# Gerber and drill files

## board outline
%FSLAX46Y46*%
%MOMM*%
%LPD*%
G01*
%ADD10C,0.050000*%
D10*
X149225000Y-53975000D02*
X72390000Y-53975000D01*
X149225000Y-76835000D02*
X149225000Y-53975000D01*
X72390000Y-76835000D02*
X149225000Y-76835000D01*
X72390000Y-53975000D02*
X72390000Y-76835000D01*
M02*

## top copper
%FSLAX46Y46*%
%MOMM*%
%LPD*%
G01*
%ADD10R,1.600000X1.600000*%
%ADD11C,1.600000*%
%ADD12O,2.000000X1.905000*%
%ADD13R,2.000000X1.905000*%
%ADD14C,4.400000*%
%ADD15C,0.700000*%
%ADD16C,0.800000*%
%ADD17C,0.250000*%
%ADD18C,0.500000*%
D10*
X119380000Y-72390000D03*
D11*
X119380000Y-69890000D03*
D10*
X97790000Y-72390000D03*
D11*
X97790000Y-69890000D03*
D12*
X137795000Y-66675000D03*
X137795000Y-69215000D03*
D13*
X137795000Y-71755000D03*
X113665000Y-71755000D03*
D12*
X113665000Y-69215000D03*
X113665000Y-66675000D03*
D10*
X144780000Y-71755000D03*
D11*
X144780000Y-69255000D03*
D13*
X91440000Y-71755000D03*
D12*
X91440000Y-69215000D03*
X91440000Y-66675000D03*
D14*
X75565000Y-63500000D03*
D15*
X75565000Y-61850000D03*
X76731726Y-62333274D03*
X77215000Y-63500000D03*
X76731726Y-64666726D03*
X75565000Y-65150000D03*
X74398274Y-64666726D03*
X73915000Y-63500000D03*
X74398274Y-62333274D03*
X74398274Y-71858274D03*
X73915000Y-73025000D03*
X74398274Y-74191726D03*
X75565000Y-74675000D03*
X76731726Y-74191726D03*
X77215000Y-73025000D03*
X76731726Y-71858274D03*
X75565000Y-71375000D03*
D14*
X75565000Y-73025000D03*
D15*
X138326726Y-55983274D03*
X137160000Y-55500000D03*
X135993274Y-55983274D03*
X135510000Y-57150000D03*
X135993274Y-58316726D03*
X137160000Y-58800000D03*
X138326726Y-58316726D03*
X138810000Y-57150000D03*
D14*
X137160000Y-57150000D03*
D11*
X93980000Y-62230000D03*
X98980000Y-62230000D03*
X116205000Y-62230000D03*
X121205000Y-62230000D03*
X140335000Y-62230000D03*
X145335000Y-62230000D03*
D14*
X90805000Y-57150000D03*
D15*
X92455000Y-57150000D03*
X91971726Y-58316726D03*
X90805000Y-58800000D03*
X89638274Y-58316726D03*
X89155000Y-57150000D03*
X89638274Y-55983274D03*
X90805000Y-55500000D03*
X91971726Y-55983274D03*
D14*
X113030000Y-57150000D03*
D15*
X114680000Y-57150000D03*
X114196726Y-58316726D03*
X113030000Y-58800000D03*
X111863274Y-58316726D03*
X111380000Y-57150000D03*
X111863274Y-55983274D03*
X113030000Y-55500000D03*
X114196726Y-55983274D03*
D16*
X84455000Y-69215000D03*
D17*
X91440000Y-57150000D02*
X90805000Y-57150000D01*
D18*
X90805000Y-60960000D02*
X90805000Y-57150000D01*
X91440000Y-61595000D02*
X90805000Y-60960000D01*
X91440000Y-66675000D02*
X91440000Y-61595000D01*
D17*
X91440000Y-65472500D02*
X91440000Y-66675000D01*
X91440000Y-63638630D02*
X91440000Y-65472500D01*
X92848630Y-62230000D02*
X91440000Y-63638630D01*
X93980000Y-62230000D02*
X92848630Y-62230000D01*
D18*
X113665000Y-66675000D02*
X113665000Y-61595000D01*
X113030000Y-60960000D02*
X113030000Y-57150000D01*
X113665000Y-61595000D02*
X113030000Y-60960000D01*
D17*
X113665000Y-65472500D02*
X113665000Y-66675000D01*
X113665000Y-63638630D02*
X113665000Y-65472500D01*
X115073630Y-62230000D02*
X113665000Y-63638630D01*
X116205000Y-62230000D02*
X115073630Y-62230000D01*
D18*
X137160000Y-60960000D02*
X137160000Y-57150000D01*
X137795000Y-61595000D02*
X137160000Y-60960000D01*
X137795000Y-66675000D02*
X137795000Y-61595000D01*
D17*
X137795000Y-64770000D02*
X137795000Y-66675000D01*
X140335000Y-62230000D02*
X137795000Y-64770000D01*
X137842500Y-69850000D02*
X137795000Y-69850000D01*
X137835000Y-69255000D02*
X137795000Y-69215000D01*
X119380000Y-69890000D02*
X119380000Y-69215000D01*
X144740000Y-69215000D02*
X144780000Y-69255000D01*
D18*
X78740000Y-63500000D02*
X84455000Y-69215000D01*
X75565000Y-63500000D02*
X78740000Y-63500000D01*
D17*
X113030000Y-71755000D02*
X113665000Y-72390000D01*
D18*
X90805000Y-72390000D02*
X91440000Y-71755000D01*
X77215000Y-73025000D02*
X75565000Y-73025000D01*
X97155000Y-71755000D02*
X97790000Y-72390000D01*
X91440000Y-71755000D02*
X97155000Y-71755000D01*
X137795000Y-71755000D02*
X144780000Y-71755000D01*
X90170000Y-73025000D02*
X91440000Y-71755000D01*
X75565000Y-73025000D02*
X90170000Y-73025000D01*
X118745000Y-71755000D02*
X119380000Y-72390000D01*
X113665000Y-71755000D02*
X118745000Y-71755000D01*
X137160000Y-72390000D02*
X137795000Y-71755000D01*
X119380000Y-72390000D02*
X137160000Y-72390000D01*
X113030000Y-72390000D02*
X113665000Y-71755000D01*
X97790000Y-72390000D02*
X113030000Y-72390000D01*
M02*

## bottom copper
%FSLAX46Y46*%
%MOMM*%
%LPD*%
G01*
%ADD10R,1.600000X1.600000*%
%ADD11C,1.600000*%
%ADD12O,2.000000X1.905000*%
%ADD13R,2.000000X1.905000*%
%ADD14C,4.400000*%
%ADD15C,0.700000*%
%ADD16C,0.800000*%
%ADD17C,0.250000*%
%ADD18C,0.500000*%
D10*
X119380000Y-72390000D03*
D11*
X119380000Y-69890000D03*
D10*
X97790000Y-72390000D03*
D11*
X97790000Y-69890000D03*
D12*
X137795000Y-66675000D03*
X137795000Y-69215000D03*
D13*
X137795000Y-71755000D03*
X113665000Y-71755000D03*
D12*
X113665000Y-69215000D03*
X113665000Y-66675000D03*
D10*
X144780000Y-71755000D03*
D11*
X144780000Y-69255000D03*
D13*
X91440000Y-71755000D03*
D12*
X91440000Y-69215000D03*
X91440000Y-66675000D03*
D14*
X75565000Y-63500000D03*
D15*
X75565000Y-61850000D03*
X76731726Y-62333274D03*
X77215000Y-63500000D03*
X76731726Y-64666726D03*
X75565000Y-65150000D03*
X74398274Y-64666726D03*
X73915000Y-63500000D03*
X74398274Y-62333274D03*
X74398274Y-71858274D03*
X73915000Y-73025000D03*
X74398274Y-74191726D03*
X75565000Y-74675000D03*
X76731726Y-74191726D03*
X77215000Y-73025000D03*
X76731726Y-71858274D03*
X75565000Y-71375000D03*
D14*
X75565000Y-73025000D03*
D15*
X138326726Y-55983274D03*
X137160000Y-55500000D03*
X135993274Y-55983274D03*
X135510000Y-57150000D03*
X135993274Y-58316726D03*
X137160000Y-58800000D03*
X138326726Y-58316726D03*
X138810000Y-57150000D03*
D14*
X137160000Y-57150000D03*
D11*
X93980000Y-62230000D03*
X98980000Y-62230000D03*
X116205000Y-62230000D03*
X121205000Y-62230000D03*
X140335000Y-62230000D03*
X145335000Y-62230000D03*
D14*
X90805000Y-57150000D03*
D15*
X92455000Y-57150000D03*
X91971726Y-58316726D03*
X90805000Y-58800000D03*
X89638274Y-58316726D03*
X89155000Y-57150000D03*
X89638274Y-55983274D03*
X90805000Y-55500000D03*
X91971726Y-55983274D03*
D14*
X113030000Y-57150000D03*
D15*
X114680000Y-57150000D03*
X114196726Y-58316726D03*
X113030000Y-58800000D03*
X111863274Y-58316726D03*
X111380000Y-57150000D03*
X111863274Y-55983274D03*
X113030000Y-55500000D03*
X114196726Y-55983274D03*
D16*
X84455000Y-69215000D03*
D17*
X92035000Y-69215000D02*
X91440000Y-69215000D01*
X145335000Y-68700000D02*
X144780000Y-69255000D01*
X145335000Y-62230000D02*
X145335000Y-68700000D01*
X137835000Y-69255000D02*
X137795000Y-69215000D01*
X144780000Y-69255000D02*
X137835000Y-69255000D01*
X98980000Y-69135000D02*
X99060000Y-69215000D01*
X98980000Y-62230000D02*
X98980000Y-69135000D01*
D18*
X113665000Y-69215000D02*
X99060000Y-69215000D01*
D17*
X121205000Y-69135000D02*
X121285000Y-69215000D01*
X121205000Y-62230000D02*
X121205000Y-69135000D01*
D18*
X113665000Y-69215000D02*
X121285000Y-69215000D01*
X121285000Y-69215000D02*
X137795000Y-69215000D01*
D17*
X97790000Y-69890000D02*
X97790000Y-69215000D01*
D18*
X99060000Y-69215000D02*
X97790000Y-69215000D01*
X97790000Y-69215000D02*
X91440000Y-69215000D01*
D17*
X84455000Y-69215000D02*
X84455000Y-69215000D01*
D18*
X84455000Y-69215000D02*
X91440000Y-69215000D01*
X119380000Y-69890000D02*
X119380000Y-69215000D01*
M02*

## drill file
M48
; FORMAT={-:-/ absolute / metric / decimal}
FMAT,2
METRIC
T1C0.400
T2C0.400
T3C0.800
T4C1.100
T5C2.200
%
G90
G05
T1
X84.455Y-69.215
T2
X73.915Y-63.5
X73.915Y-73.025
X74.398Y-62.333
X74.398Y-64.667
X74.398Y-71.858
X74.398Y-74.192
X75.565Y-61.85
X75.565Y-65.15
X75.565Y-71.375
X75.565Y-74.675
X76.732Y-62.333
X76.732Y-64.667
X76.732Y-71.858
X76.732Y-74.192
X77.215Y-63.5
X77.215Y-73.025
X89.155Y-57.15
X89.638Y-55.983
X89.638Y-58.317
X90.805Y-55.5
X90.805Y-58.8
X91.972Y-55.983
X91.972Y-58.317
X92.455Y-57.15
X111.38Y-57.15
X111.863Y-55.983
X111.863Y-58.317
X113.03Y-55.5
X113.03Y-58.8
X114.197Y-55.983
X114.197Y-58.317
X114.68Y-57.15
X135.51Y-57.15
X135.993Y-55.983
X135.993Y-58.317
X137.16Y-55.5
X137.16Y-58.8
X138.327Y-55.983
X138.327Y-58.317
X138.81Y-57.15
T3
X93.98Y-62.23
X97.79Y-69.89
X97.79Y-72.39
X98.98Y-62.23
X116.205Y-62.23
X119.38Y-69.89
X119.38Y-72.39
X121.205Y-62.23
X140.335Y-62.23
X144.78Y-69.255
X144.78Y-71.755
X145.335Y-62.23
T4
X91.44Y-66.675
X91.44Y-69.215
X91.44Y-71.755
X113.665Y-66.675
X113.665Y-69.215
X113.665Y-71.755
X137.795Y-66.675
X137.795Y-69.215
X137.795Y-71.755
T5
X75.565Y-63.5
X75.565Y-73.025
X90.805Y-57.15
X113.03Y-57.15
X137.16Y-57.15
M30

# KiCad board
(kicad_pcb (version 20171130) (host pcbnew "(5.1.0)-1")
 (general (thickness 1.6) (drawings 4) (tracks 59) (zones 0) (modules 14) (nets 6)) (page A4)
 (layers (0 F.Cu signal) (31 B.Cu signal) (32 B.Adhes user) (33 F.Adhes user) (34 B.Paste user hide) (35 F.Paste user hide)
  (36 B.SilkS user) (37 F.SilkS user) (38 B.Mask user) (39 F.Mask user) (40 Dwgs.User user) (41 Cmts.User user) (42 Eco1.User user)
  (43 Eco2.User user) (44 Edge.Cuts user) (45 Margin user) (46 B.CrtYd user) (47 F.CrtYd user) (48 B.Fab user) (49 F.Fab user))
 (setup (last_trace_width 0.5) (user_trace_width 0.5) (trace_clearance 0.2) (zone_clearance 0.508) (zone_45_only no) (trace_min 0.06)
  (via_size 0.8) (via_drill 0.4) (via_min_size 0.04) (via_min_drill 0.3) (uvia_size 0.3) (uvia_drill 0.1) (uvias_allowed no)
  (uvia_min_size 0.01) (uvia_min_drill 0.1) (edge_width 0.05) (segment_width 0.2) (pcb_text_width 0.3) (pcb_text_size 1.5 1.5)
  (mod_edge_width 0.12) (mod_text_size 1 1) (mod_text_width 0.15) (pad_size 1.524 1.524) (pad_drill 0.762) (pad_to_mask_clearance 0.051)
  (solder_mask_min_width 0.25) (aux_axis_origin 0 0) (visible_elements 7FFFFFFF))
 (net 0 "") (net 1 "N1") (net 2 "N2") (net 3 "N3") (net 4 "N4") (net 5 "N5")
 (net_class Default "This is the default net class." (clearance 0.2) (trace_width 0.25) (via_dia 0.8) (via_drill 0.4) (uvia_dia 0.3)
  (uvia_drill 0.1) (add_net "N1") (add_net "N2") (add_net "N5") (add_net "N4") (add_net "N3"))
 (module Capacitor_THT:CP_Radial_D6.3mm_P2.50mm (layer F.Cu) (at 119.38 72.39 90)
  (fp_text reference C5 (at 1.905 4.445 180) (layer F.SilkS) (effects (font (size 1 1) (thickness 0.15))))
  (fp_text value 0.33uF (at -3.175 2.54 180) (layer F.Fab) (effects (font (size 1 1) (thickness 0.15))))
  (pad 1 thru_hole rect (at 0 0 90) (size 1.6 1.6) (drill 0.8) (layers *.Cu *.Mask) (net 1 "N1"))
  (pad 2 thru_hole circle (at 2.5 0 90) (size 1.6 1.6) (drill 0.8) (layers *.Cu *.Mask) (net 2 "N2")))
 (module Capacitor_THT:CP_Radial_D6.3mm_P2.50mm (layer F.Cu) (at 97.79 72.39 90)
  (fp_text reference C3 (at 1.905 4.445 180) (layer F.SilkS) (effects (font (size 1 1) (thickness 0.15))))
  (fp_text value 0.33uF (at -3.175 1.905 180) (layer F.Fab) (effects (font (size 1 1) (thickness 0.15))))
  (pad 1 thru_hole rect (at 0 0 90) (size 1.6 1.6) (drill 0.8) (layers *.Cu *.Mask) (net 1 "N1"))
  (pad 2 thru_hole circle (at 2.5 0 90) (size 1.6 1.6) (drill 0.8) (layers *.Cu *.Mask) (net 2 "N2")))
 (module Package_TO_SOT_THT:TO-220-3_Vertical (layer F.Cu) (at 137.795 71.755 90)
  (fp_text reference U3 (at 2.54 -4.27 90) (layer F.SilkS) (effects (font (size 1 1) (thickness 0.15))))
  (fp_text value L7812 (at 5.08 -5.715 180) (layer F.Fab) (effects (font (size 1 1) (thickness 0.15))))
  (pad 3 thru_hole oval (at 5.08 0 90) (size 1.905 2) (drill 1.1) (layers *.Cu *.Mask) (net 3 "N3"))
  (pad 2 thru_hole oval (at 2.54 0 90) (size 1.905 2) (drill 1.1) (layers *.Cu *.Mask) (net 2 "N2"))
  (pad 1 thru_hole rect (at 0 0 90) (size 1.905 2) (drill 1.1) (layers *.Cu *.Mask) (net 1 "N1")))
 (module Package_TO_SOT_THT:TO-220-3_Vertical (layer F.Cu) (at 113.665 71.755 90)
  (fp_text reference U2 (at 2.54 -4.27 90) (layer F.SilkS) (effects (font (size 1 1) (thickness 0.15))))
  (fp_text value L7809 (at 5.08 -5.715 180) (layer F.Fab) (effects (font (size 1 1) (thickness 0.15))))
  (pad 1 thru_hole rect (at 0 0 90) (size 1.905 2) (drill 1.1) (layers *.Cu *.Mask) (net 1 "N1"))
  (pad 2 thru_hole oval (at 2.54 0 90) (size 1.905 2) (drill 1.1) (layers *.Cu *.Mask) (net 2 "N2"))
  (pad 3 thru_hole oval (at 5.08 0 90) (size 1.905 2) (drill 1.1) (layers *.Cu *.Mask) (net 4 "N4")))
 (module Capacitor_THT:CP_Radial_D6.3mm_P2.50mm (layer F.Cu) (at 144.78 71.755 90)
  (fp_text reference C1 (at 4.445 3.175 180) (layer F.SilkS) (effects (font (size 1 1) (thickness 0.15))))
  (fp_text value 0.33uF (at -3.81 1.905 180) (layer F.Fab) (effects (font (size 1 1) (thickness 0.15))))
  (pad 1 thru_hole rect (at 0 0 90) (size 1.6 1.6) (drill 0.8) (layers *.Cu *.Mask) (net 1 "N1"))
  (pad 2 thru_hole circle (at 2.5 0 90) (size 1.6 1.6) (drill 0.8) (layers *.Cu *.Mask) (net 2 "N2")))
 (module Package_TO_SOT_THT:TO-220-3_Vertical (layer F.Cu) (at 91.44 71.755 90)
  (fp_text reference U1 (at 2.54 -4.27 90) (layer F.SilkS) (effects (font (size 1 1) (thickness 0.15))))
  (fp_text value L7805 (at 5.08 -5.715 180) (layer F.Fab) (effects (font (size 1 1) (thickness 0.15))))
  (pad 1 thru_hole rect (at 0 0 90) (size 1.905 2) (drill 1.1) (layers *.Cu *.Mask) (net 1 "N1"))
  (pad 2 thru_hole oval (at 2.54 0 90) (size 1.905 2) (drill 1.1) (layers *.Cu *.Mask) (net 2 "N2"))
  (pad 3 thru_hole oval (at 5.08 0 90) (size 1.905 2) (drill 1.1) (layers *.Cu *.Mask) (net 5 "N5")))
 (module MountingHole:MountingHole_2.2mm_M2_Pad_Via (layer F.Cu) (at 75.565 63.5 90)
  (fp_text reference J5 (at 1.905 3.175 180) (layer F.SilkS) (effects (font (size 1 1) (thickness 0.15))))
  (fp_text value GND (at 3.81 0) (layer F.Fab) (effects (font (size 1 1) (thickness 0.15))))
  (pad 1 thru_hole circle (at 0 0 90) (size 4.4 4.4) (drill 2.2) (layers *.Cu *.Mask) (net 2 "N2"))
  (pad 1 thru_hole circle (at 1.65 0 90) (size 0.7 0.7) (drill 0.4) (layers *.Cu *.Mask) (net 2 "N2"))
  (pad 1 thru_hole circle (at 1.166726 1.166726 90) (size 0.7 0.7) (drill 0.4) (layers *.Cu *.Mask) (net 2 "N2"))
  (pad 1 thru_hole circle (at 0 1.65 90) (size 0.7 0.7) (drill 0.4) (layers *.Cu *.Mask) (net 2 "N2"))
  (pad 1 thru_hole circle (at -1.166726 1.166726 90) (size 0.7 0.7) (drill 0.4) (layers *.Cu *.Mask) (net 2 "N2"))
  (pad 1 thru_hole circle (at -1.65 0 90) (size 0.7 0.7) (drill 0.4) (layers *.Cu *.Mask) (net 2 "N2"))
  (pad 1 thru_hole circle (at -1.166726 -1.166726 90) (size 0.7 0.7) (drill 0.4) (layers *.Cu *.Mask) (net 2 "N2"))
  (pad 1 thru_hole circle (at 0 -1.65 90) (size 0.7 0.7) (drill 0.4) (layers *.Cu *.Mask) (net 2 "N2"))
  (pad 1 thru_hole circle (at 1.166726 -1.166726 90) (size 0.7 0.7) (drill 0.4) (layers *.Cu *.Mask) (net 2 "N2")))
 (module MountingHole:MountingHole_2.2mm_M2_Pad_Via (layer F.Cu) (at 75.565 73.025 90)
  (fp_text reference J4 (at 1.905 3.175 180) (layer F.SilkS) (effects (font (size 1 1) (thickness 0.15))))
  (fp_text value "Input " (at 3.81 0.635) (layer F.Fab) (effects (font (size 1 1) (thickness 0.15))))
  (pad 1 thru_hole circle (at 1.166726 -1.166726 90) (size 0.7 0.7) (drill 0.4) (layers *.Cu *.Mask) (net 1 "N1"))
  (pad 1 thru_hole circle (at 0 -1.65 90) (size 0.7 0.7) (drill 0.4) (layers *.Cu *.Mask) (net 1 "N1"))
  (pad 1 thru_hole circle (at -1.166726 -1.166726 90) (size 0.7 0.7) (drill 0.4) (layers *.Cu *.Mask) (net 1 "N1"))
  (pad 1 thru_hole circle (at -1.65 0 90) (size 0.7 0.7) (drill 0.4) (layers *.Cu *.Mask) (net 1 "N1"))
  (pad 1 thru_hole circle (at -1.166726 1.166726 90) (size 0.7 0.7) (drill 0.4) (layers *.Cu *.Mask) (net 1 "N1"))
  (pad 1 thru_hole circle (at 0 1.65 90) (size 0.7 0.7) (drill 0.4) (layers *.Cu *.Mask) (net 1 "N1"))
  (pad 1 thru_hole circle (at 1.166726 1.166726 90) (size 0.7 0.7) (drill 0.4) (layers *.Cu *.Mask) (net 1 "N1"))
  (pad 1 thru_hole circle (at 1.65 0 90) (size 0.7 0.7) (drill 0.4) (layers *.Cu *.Mask) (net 1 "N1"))
  (pad 1 thru_hole circle (at 0 0 90) (size 4.4 4.4) (drill 2.2) (layers *.Cu *.Mask) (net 1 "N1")))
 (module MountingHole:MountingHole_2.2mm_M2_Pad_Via (layer F.Cu) (at 137.16 57.15)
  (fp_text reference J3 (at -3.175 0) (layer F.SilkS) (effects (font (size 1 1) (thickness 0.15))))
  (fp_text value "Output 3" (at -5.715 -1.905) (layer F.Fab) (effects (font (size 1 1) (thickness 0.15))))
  (pad 1 thru_hole circle (at 1.166726 -1.166726) (size 0.7 0.7) (drill 0.4) (layers *.Cu *.Mask) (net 3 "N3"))
  (pad 1 thru_hole circle (at 0 -1.65) (size 0.7 0.7) (drill 0.4) (layers *.Cu *.Mask) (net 3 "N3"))
  (pad 1 thru_hole circle (at -1.166726 -1.166726) (size 0.7 0.7) (drill 0.4) (layers *.Cu *.Mask) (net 3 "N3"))
  (pad 1 thru_hole circle (at -1.65 0) (size 0.7 0.7) (drill 0.4) (layers *.Cu *.Mask) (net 3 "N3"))
  (pad 1 thru_hole circle (at -1.166726 1.166726) (size 0.7 0.7) (drill 0.4) (layers *.Cu *.Mask) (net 3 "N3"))
  (pad 1 thru_hole circle (at 0 1.65) (size 0.7 0.7) (drill 0.4) (layers *.Cu *.Mask) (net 3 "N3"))
  (pad 1 thru_hole circle (at 1.166726 1.166726) (size 0.7 0.7) (drill 0.4) (layers *.Cu *.Mask) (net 3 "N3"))
  (pad 1 thru_hole circle (at 1.65 0) (size 0.7 0.7) (drill 0.4) (layers *.Cu *.Mask) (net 3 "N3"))
  (pad 1 thru_hole circle (at 0 0) (size 4.4 4.4) (drill 2.2) (layers *.Cu *.Mask) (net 3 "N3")))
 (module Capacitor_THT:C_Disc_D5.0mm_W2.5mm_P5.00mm (layer F.Cu) (at 93.98 62.23)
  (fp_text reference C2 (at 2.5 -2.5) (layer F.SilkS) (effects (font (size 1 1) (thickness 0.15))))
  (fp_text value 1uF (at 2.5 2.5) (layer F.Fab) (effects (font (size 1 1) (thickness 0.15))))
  (pad 1 thru_hole circle (at 0 0) (size 1.6 1.6) (drill 0.8) (layers *.Cu *.Mask) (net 5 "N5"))
  (pad 2 thru_hole circle (at 5 0) (size 1.6 1.6) (drill 0.8) (layers *.Cu *.Mask) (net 2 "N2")))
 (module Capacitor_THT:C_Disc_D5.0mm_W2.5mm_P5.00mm (layer F.Cu) (at 116.205 62.23)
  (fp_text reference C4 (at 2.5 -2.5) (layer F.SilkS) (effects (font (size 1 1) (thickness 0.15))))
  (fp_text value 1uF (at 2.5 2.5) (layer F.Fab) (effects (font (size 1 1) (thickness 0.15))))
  (pad 1 thru_hole circle (at 0 0) (size 1.6 1.6) (drill 0.8) (layers *.Cu *.Mask) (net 4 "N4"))
  (pad 2 thru_hole circle (at 5 0) (size 1.6 1.6) (drill 0.8) (layers *.Cu *.Mask) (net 2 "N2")))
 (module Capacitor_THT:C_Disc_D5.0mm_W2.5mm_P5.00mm (layer F.Cu) (at 140.335 62.23)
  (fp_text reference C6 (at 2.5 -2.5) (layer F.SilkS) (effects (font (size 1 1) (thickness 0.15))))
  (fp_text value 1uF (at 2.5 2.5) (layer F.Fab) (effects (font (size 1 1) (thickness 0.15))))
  (pad 1 thru_hole circle (at 0 0) (size 1.6 1.6) (drill 0.8) (layers *.Cu *.Mask) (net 3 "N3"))
  (pad 2 thru_hole circle (at 5 0) (size 1.6 1.6) (drill 0.8) (layers *.Cu *.Mask) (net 2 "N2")))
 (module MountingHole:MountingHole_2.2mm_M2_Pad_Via (layer F.Cu) (at 90.805 57.15)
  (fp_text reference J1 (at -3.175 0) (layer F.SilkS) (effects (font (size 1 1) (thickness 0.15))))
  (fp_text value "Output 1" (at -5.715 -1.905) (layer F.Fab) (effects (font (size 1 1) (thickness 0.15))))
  (pad 1 thru_hole circle (at 0 0) (size 4.4 4.4) (drill 2.2) (layers *.Cu *.Mask) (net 5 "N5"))
  (pad 1 thru_hole circle (at 1.65 0) (size 0.7 0.7) (drill 0.4) (layers *.Cu *.Mask) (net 5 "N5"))
  (pad 1 thru_hole circle (at 1.166726 1.166726) (size 0.7 0.7) (drill 0.4) (layers *.Cu *.Mask) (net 5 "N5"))
  (pad 1 thru_hole circle (at 0 1.65) (size 0.7 0.7) (drill 0.4) (layers *.Cu *.Mask) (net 5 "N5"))
  (pad 1 thru_hole circle (at -1.166726 1.166726) (size 0.7 0.7) (drill 0.4) (layers *.Cu *.Mask) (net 5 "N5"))
  (pad 1 thru_hole circle (at -1.65 0) (size 0.7 0.7) (drill 0.4) (layers *.Cu *.Mask) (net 5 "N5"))
  (pad 1 thru_hole circle (at -1.166726 -1.166726) (size 0.7 0.7) (drill 0.4) (layers *.Cu *.Mask) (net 5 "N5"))
  (pad 1 thru_hole circle (at 0 -1.65) (size 0.7 0.7) (drill 0.4) (layers *.Cu *.Mask) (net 5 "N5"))
  (pad 1 thru_hole circle (at 1.166726 -1.166726) (size 0.7 0.7) (drill 0.4) (layers *.Cu *.Mask) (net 5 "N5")))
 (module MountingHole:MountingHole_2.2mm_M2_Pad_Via (layer F.Cu) (at 113.03 57.15)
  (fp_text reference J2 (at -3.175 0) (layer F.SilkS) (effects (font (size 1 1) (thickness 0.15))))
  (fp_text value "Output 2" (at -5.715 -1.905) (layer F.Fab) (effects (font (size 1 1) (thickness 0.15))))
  (pad 1 thru_hole circle (at 0 0) (size 4.4 4.4) (drill 2.2) (layers *.Cu *.Mask) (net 4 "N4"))
  (pad 1 thru_hole circle (at 1.65 0) (size 0.7 0.7) (drill 0.4) (layers *.Cu *.Mask) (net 4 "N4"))
  (pad 1 thru_hole circle (at 1.166726 1.166726) (size 0.7 0.7) (drill 0.4) (layers *.Cu *.Mask) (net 4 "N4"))
  (pad 1 thru_hole circle (at 0 1.65) (size 0.7 0.7) (drill 0.4) (layers *.Cu *.Mask) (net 4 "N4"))
  (pad 1 thru_hole circle (at -1.166726 1.166726) (size 0.7 0.7) (drill 0.4) (layers *.Cu *.Mask) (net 4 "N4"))
  (pad 1 thru_hole circle (at -1.65 0) (size 0.7 0.7) (drill 0.4) (layers *.Cu *.Mask) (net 4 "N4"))
  (pad 1 thru_hole circle (at -1.166726 -1.166726) (size 0.7 0.7) (drill 0.4) (layers *.Cu *.Mask) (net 4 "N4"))
  (pad 1 thru_hole circle (at 0 -1.65) (size 0.7 0.7) (drill 0.4) (layers *.Cu *.Mask) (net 4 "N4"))
  (pad 1 thru_hole circle (at 1.166726 -1.166726) (size 0.7 0.7) (drill 0.4) (layers *.Cu *.Mask) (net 4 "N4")))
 (gr_line (start 149.225 53.975) (end 72.39 53.975) (layer Edge.Cuts) (width 0.05))
 (gr_line (start 149.225 76.835) (end 149.225 53.975) (layer Edge.Cuts) (width 0.05))
 (gr_line (start 72.39 76.835) (end 149.225 76.835) (layer Edge.Cuts) (width 0.05))
 (gr_line (start 72.39 53.975) (end 72.39 76.835) (layer Edge.Cuts) (width 0.05))
 (segment (start 91.44 57.15) (end 90.805 57.15) (width 0.25) (layer F.Cu) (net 5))
 (segment (start 90.805 60.96) (end 90.805 57.15) (width 0.5) (layer F.Cu) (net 5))
 (segment (start 91.44 61.595) (end 90.805 60.96) (width 0.5) (layer F.Cu) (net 5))
 (segment (start 91.44 66.675) (end 91.44 61.595) (width 0.5) (layer F.Cu) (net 5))
 (segment (start 91.44 65.4725) (end 91.44 66.675) (width 0.25) (layer F.Cu) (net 5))
 (segment (start 91.44 63.63863) (end 91.44 65.4725) (width 0.25) (layer F.Cu) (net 5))
 (segment (start 92.84863 62.23) (end 91.44 63.63863) (width 0.25) (layer F.Cu) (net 5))
 (segment (start 93.98 62.23) (end 92.84863 62.23) (width 0.25) (layer F.Cu) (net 5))
 (segment (start 113.665 66.675) (end 113.665 61.595) (width 0.5) (layer F.Cu) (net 4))
 (segment (start 113.03 60.96) (end 113.03 57.15) (width 0.5) (layer F.Cu) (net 4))
 (segment (start 113.665 61.595) (end 113.03 60.96) (width 0.5) (layer F.Cu) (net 4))
 (segment (start 113.665 65.4725) (end 113.665 66.675) (width 0.25) (layer F.Cu) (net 4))
 (segment (start 113.665 63.63863) (end 113.665 65.4725) (width 0.25) (layer F.Cu) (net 4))
 (segment (start 115.07363 62.23) (end 113.665 63.63863) (width 0.25) (layer F.Cu) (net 4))
 (segment (start 116.205 62.23) (end 115.07363 62.23) (width 0.25) (layer F.Cu) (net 4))
 (segment (start 137.16 60.96) (end 137.16 57.15) (width 0.5) (layer F.Cu) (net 3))
 (segment (start 137.795 61.595) (end 137.16 60.96) (width 0.5) (layer F.Cu) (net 3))
 (segment (start 137.795 66.675) (end 137.795 61.595) (width 0.5) (layer F.Cu) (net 3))
 (segment (start 137.795 64.77) (end 137.795 66.675) (width 0.25) (layer F.Cu) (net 3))
 (segment (start 140.335 62.23) (end 137.795 64.77) (width 0.25) (layer F.Cu) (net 3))
 (segment (start 137.8425 69.85) (end 137.795 69.85) (width 0.25) (layer F.Cu) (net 2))
 (segment (start 92.035 69.215) (end 91.44 69.215) (width 0.25) (layer B.Cu) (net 2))
 (segment (start 137.835 69.255) (end 137.795 69.215) (width 0.25) (layer F.Cu) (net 2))
 (segment (start 119.38 69.89) (end 119.38 69.215) (width 0.25) (layer F.Cu) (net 2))
 (segment (start 144.74 69.215) (end 144.78 69.255) (width 0.25) (layer F.Cu) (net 2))
 (segment (start 145.335 68.7) (end 144.78 69.255) (width 0.25) (layer B.Cu) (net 2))
 (segment (start 145.335 62.23) (end 145.335 68.7) (width 0.25) (layer B.Cu) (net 2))
 (segment (start 137.835 69.255) (end 137.795 69.215) (width 0.25) (layer B.Cu) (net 2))
 (segment (start 144.78 69.255) (end 137.835 69.255) (width 0.25) (layer B.Cu) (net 2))
 (segment (start 98.98 69.135) (end 99.06 69.215) (width 0.25) (layer B.Cu) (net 2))
 (segment (start 98.98 62.23) (end 98.98 69.135) (width 0.25) (layer B.Cu) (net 2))
 (segment (start 113.665 69.215) (end 99.06 69.215) (width 0.5) (layer B.Cu) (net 2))
 (segment (start 121.205 69.135) (end 121.285 69.215) (width 0.25) (layer B.Cu) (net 2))
 (segment (start 121.205 62.23) (end 121.205 69.135) (width 0.25) (layer B.Cu) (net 2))
 (segment (start 113.665 69.215) (end 121.285 69.215) (width 0.5) (layer B.Cu) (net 2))
 (segment (start 121.285 69.215) (end 137.795 69.215) (width 0.5) (layer B.Cu) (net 2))
 (segment (start 97.79 69.89) (end 97.79 69.215) (width 0.25) (layer B.Cu) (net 2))
 (segment (start 99.06 69.215) (end 97.79 69.215) (width 0.5) (layer B.Cu) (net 2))
 (segment (start 97.79 69.215) (end 91.44 69.215) (width 0.5) (layer B.Cu) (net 2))
 (segment (start 84.455 69.215) (end 84.455 69.215) (width 0.25) (layer B.Cu) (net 2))
 (via (at 84.455 69.215) (size 0.8) (drill 0.4) (layers F.Cu B.Cu) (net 2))
 (segment (start 84.455 69.215) (end 91.44 69.215) (width 0.5) (layer B.Cu) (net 2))
 (segment (start 78.74 63.5) (end 84.455 69.215) (width 0.5) (layer F.Cu) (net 2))
 (segment (start 75.565 63.5) (end 78.74 63.5) (width 0.5) (layer F.Cu) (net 2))
 (segment (start 119.38 69.89) (end 119.38 69.215) (width 0.5) (layer B.Cu) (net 2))
 (segment (start 113.03 71.755) (end 113.665 72.39) (width 0.25) (layer F.Cu) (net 1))
 (segment (start 90.805 72.39) (end 91.44 71.755) (width 0.5) (layer F.Cu) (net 1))
 (segment (start 77.215 73.025) (end 75.565 73.025) (width 0.5) (layer F.Cu) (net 1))
 (segment (start 97.155 71.755) (end 97.79 72.39) (width 0.5) (layer F.Cu) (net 1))
 (segment (start 91.44 71.755) (end 97.155 71.755) (width 0.5) (layer F.Cu) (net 1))
 (segment (start 137.795 71.755) (end 144.78 71.755) (width 0.5) (layer F.Cu) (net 1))
 (segment (start 90.17 73.025) (end 91.44 71.755) (width 0.5) (layer F.Cu) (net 1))
 (segment (start 75.565 73.025) (end 90.17 73.025) (width 0.5) (layer F.Cu) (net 1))
 (segment (start 118.745 71.755) (end 119.38 72.39) (width 0.5) (layer F.Cu) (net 1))
 (segment (start 113.665 71.755) (end 118.745 71.755) (width 0.5) (layer F.Cu) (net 1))
 (segment (start 137.16 72.39) (end 137.795 71.755) (width 0.5) (layer F.Cu) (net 1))
 (segment (start 119.38 72.39) (end 137.16 72.39) (width 0.5) (layer F.Cu) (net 1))
 (segment (start 113.03 72.39) (end 113.665 71.755) (width 0.5) (layer F.Cu) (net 1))
 (segment (start 97.79 72.39) (end 113.03 72.39) (width 0.5) (layer F.Cu) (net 1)))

